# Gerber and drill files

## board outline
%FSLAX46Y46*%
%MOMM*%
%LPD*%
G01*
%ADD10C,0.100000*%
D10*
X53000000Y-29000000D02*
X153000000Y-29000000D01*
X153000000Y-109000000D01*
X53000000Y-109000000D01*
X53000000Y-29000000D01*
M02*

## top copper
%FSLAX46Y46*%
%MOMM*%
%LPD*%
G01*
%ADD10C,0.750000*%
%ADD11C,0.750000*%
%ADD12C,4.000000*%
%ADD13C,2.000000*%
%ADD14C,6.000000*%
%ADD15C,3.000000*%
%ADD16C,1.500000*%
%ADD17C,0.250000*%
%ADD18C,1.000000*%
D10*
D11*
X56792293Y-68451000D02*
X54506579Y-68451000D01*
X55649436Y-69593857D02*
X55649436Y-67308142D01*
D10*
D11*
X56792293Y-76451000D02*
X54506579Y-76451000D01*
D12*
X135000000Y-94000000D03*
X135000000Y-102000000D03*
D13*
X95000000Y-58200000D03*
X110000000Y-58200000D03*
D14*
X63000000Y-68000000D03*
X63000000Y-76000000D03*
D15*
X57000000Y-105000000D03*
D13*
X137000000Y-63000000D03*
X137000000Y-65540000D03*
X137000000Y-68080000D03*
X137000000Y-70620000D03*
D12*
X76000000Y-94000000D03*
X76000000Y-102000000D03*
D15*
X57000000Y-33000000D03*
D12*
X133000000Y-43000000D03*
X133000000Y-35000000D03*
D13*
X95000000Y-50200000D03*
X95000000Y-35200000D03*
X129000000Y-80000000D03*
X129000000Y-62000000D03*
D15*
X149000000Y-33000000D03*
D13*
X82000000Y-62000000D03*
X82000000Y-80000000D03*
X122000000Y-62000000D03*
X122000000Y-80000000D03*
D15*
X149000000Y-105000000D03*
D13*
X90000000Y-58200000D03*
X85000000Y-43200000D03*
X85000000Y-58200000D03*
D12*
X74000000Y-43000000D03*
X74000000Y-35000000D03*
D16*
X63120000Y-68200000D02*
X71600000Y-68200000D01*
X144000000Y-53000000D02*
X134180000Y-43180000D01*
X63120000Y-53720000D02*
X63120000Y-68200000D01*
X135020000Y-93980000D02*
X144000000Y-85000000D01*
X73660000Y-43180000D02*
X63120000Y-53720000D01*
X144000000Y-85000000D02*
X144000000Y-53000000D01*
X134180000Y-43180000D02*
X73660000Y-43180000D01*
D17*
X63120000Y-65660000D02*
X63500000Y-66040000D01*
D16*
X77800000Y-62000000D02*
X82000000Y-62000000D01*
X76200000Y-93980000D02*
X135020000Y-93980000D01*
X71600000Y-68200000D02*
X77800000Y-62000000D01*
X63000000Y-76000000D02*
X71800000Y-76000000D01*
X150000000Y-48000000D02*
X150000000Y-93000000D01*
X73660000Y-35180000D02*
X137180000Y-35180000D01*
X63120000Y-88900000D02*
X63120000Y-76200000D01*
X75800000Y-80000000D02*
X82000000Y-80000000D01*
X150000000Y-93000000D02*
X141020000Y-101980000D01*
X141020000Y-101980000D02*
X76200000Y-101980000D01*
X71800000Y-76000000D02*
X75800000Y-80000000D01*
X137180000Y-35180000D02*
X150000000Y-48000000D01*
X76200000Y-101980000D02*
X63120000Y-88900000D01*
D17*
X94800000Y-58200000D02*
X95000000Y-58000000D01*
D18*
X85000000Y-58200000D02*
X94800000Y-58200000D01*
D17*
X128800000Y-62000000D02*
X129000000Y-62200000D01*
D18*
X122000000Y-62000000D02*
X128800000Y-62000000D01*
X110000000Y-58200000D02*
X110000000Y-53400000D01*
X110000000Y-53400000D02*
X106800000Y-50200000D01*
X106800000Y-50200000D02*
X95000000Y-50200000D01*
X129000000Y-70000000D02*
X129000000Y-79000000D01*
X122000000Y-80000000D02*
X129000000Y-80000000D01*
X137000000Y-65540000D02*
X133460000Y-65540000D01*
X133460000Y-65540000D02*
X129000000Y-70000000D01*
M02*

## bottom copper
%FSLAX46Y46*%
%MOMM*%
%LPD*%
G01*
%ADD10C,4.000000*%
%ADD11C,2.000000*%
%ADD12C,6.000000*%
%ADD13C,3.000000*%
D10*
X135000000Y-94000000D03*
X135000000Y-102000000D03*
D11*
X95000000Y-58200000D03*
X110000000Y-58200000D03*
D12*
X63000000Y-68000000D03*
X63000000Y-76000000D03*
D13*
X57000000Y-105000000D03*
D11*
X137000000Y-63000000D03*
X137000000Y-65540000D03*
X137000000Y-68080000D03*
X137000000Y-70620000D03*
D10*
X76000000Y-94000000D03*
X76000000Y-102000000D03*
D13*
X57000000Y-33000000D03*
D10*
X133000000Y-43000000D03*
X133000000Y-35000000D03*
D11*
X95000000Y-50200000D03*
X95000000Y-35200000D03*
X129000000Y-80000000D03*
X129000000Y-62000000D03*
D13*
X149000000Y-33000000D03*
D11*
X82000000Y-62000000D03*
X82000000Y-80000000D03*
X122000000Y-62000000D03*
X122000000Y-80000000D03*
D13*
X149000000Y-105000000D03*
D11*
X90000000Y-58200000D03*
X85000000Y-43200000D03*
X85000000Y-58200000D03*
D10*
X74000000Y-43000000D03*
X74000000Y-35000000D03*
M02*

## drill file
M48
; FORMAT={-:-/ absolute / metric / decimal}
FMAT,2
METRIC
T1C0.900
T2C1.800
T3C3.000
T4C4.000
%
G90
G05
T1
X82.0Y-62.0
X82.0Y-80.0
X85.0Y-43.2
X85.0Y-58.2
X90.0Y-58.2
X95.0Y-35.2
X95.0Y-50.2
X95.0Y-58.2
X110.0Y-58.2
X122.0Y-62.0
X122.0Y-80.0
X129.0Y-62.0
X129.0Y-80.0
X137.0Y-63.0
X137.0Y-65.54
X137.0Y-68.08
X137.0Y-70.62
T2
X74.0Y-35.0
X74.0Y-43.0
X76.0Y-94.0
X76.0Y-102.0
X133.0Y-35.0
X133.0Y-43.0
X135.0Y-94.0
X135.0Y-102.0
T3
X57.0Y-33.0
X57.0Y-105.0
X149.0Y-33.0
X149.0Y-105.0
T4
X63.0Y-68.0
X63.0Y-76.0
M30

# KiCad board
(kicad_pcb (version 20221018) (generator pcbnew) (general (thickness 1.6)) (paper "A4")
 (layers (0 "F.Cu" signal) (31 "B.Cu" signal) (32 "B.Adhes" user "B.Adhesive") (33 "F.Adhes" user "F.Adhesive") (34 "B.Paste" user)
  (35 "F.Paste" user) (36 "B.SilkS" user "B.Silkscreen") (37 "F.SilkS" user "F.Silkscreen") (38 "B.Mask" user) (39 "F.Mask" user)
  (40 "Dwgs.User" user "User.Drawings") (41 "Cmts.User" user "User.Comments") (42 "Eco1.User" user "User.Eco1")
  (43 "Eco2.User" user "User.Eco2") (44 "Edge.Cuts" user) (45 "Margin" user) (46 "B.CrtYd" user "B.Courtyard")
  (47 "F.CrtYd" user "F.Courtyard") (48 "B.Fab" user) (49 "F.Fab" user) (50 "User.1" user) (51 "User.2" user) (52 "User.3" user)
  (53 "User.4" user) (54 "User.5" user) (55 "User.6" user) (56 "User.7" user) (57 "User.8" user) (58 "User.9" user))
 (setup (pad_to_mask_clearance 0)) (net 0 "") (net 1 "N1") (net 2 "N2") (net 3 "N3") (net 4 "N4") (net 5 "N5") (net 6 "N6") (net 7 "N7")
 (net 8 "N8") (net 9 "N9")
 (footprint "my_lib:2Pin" (layer "F.Cu") (at 135 94)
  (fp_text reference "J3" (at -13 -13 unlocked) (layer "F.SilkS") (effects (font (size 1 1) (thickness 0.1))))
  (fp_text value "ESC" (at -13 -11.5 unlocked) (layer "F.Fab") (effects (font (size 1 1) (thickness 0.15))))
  (pad "1" thru_hole circle (at 0 0) (size 4 4) (drill 1.8) (layers "*.Cu" "*.Mask") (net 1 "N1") (clearance 0.5))
  (pad "2" thru_hole circle (at 0 8) (size 4 4) (drill 1.8) (layers "*.Cu" "*.Mask") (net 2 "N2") (clearance 0.5)))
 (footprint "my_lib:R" (layer "F.Cu") (at 95 58.2)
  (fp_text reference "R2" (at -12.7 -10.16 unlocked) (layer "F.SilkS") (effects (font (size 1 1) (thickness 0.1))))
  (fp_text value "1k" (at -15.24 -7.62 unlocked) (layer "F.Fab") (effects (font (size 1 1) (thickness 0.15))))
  (pad "1" thru_hole circle (at 0 0) (size 2 2) (drill 0.9) (layers "*.Cu" "*.Mask") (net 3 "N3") (clearance 0.5))
  (pad "2" thru_hole circle (at 15 0) (size 2 2) (drill 0.9) (layers "*.Cu" "*.Mask") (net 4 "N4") (clearance 0.5)))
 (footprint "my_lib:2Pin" (layer "F.Cu") (at 63 68)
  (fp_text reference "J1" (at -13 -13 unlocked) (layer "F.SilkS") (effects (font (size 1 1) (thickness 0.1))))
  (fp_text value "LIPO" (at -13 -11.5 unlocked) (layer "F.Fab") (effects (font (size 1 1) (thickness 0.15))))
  (pad "1" thru_hole circle (at 0 0) (size 6 6) (drill 4) (layers "*.Cu" "*.Mask") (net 1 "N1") (clearance 0.5))
  (pad "2" thru_hole circle (at 0 8) (size 6 6) (drill 4) (layers "*.Cu" "*.Mask") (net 2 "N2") (clearance 0.5)))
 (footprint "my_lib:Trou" (layer "F.Cu") (at 57 105)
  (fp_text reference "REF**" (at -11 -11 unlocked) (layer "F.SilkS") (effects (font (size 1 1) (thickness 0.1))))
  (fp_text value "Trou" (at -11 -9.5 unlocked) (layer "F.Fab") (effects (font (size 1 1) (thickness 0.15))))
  (pad "1" thru_hole circle (at 0 0) (size 3 3) (drill 3) (layers "*.Cu" "*.Mask")))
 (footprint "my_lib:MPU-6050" (layer "F.Cu") (at 137 63)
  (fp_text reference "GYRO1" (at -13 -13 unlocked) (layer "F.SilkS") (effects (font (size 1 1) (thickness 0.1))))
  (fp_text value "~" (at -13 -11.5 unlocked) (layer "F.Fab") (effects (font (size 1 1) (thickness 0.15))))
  (pad "1" thru_hole circle (at 0 0) (size 2 2) (drill 0.9) (layers "*.Cu" "*.Mask") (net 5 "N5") (clearance 0.5))
  (pad "2" thru_hole circle (at 0 2.54) (size 2 2) (drill 0.9) (layers "*.Cu" "*.Mask") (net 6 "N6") (clearance 0.5))
  (pad "3" thru_hole circle (at 0 5.08) (size 2 2) (drill 0.9) (layers "*.Cu" "*.Mask") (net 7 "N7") (clearance 0.5))
  (pad "4" thru_hole circle (at 0 7.62) (size 2 2) (drill 0.9) (layers "*.Cu" "*.Mask") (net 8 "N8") (clearance 0.5)))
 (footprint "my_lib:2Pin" (layer "F.Cu") (at 76 94)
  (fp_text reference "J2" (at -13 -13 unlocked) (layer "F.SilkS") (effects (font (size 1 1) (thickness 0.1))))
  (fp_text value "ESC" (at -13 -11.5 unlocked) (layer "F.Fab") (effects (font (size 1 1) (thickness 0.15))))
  (pad "1" thru_hole circle (at 0 0) (size 4 4) (drill 1.8) (layers "*.Cu" "*.Mask") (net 1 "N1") (clearance 0.5))
  (pad "2" thru_hole circle (at 0 8) (size 4 4) (drill 1.8) (layers "*.Cu" "*.Mask") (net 2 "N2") (clearance 0.5)))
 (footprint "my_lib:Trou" (layer "F.Cu") (at 57 33)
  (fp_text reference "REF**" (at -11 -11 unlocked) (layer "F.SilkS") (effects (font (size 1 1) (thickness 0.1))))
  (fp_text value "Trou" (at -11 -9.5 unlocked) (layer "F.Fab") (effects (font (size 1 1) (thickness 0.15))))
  (pad "1" thru_hole circle (at 0 0) (size 3 3) (drill 3) (layers "*.Cu" "*.Mask")))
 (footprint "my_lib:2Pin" (layer "F.Cu") (at 133 43 180)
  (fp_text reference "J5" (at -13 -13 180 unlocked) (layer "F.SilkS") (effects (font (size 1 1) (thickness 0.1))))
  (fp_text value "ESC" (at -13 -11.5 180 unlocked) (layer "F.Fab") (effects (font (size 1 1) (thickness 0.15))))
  (pad "1" thru_hole circle (at 0 0 180) (size 4 4) (drill 1.8) (layers "*.Cu" "*.Mask") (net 1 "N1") (clearance 0.5))
  (pad "2" thru_hole circle (at 0 8 180) (size 4 4) (drill 1.8) (layers "*.Cu" "*.Mask") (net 2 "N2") (clearance 0.5)))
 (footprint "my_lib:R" (layer "F.Cu") (at 95 50.2 90)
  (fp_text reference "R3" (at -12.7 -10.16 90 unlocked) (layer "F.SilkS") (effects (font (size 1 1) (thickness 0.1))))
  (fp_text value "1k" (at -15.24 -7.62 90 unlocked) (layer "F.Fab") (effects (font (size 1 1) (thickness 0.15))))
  (pad "1" thru_hole circle (at 0 0 90) (size 2 2) (drill 0.9) (layers "*.Cu" "*.Mask") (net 4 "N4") (clearance 0.5))
  (pad "2" thru_hole circle (at 15 0 90) (size 2 2) (drill 0.9) (layers "*.Cu" "*.Mask") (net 2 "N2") (clearance 0.5)))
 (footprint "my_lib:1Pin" (layer "F.Cu") (at 129 80)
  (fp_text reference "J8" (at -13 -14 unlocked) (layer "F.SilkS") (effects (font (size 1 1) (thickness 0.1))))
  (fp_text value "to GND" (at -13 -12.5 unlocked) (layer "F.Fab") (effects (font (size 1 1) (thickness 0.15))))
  (pad "1" thru_hole circle (at 0 0) (size 2 2) (drill 0.9) (layers "*.Cu" "*.Mask") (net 6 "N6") (clearance 0.5)))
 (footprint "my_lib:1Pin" (layer "F.Cu") (at 129 62)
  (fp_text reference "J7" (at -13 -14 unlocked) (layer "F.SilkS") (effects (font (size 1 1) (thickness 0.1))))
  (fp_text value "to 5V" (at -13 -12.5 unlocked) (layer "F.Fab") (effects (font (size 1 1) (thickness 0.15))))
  (pad "1" thru_hole circle (at 0 0) (size 2 2) (drill 0.9) (layers "*.Cu" "*.Mask") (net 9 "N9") (clearance 0.5)))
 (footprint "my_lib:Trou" (layer "F.Cu") (at 149 33)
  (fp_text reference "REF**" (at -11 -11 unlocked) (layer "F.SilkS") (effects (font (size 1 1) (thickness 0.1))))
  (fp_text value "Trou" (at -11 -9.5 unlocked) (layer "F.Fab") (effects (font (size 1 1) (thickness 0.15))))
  (pad "1" thru_hole circle (at 0 0) (size 3 3) (drill 3) (layers "*.Cu" "*.Mask")))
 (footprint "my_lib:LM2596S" (layer "F.Cu") (at 82 62)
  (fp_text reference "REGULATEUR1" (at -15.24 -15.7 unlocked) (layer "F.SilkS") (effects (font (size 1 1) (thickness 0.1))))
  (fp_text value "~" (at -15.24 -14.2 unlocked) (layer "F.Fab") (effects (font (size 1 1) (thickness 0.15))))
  (pad "1" thru_hole circle (at 0 0) (size 2 2) (drill 0.9) (layers "*.Cu" "*.Mask") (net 1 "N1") (clearance 0.5))
  (pad "2" thru_hole circle (at 0 18) (size 2 2) (drill 0.9) (layers "*.Cu" "*.Mask") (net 2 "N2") (clearance 0.5))
  (pad "3" thru_hole circle (at 40 0) (size 2 2) (drill 0.9) (layers "*.Cu" "*.Mask") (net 9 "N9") (clearance 0.5))
  (pad "4" thru_hole circle (at 40 18) (size 2 2) (drill 0.9) (layers "*.Cu" "*.Mask") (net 6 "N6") (clearance 0.5)))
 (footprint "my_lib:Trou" (layer "F.Cu") (at 149 105)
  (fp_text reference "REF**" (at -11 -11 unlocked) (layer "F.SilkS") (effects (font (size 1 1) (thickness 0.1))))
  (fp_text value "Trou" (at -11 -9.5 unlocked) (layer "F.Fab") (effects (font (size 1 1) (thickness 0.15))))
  (pad "1" thru_hole circle (at 0 0) (size 3 3) (drill 3) (layers "*.Cu" "*.Mask")))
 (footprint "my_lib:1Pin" (layer "F.Cu") (at 90 58.2)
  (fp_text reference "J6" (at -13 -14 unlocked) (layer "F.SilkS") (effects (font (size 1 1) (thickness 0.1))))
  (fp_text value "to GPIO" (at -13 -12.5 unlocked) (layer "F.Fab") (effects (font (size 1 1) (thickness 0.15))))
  (pad "1" thru_hole circle (at 0 0) (size 2 2) (drill 0.9) (layers "*.Cu" "*.Mask") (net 3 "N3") (clearance 0.5)))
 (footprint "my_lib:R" (layer "B.Cu") (at 85 43.2 -90)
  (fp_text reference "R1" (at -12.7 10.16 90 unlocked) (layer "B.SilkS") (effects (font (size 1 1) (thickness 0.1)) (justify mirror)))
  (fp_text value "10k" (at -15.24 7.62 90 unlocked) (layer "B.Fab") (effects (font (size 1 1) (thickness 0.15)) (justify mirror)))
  (pad "1" thru_hole circle (at 0 0 270) (size 2 2) (drill 0.9) (layers "*.Cu" "*.Mask") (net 1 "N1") (clearance 0.5))
  (pad "2" thru_hole circle (at 15 0 270) (size 2 2) (drill 0.9) (layers "*.Cu" "*.Mask") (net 3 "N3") (clearance 0.5)))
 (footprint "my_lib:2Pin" (layer "B.Cu") (at 74 43)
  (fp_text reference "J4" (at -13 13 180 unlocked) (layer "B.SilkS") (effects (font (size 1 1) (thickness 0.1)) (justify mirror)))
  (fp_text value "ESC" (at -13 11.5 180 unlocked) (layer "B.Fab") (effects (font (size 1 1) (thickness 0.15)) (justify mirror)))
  (pad "1" thru_hole circle (at 0 0) (size 4 4) (drill 1.8) (layers "*.Cu" "*.Mask") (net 1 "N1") (clearance 0.5))
  (pad "2" thru_hole circle (at 0 -8) (size 4 4) (drill 1.8) (layers "*.Cu" "*.Mask") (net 2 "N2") (clearance 0.5)))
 (gr_rect (start 53 29) (end 153 109) (stroke (width 0.1) (type default)) (fill none) (layer "Edge.Cuts"))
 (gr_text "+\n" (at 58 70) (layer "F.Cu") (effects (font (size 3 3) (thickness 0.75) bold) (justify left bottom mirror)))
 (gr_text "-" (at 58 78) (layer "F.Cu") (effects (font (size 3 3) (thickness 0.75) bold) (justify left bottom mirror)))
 (segment (start 63.12 68.2) (end 71.6 68.2) (width 1.5) (layer "F.Cu") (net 1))
 (segment (start 144 53) (end 134.18 43.18) (width 1.5) (layer "F.Cu") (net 1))
 (segment (start 63.12 53.72) (end 63.12 68.2) (width 1.5) (layer "F.Cu") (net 1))
 (segment (start 135.02 93.98) (end 144 85) (width 1.5) (layer "F.Cu") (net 1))
 (segment (start 73.66 43.18) (end 63.12 53.72) (width 1.5) (layer "F.Cu") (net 1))
 (segment (start 144 85) (end 144 53) (width 1.5) (layer "F.Cu") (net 1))
 (segment (start 134.18 43.18) (end 73.66 43.18) (width 1.5) (layer "F.Cu") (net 1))
 (segment (start 63.12 65.66) (end 63.5 66.04) (width 0.25) (layer "F.Cu") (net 1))
 (segment (start 77.8 62) (end 82 62) (width 1.5) (layer "F.Cu") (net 1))
 (segment (start 76.2 93.98) (end 135.02 93.98) (width 1.5) (layer "F.Cu") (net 1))
 (segment (start 71.6 68.2) (end 77.8 62) (width 1.5) (layer "F.Cu") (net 1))
 (segment (start 63 76) (end 71.8 76) (width 1.5) (layer "F.Cu") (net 2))
 (segment (start 150 48) (end 150 93) (width 1.5) (layer "F.Cu") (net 2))
 (segment (start 73.66 35.18) (end 137.18 35.18) (width 1.5) (layer "F.Cu") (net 2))
 (segment (start 63.12 88.9) (end 63.12 76.2) (width 1.5) (layer "F.Cu") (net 2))
 (segment (start 75.8 80) (end 82 80) (width 1.5) (layer "F.Cu") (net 2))
 (segment (start 150 93) (end 141.02 101.98) (width 1.5) (layer "F.Cu") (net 2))
 (segment (start 141.02 101.98) (end 76.2 101.98) (width 1.5) (layer "F.Cu") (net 2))
 (segment (start 71.8 76) (end 75.8 80) (width 1.5) (layer "F.Cu") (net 2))
 (segment (start 137.18 35.18) (end 150 48) (width 1.5) (layer "F.Cu") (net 2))
 (segment (start 76.2 101.98) (end 63.12 88.9) (width 1.5) (layer "F.Cu") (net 2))
 (segment (start 94.8 58.2) (end 95 58) (width 0.25) (layer "F.Cu") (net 3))
 (segment (start 85 58.2) (end 94.8 58.2) (width 1) (layer "F.Cu") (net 3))
 (segment (start 128.8 62) (end 129 62.2) (width 0.25) (layer "F.Cu") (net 9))
 (segment (start 122 62) (end 128.8 62) (width 1) (layer "F.Cu") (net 9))
 (segment (start 110 58.2) (end 110 53.4) (width 1) (layer "F.Cu") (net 4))
 (segment (start 110 53.4) (end 106.8 50.2) (width 1) (layer "F.Cu") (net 4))
 (segment (start 106.8 50.2) (end 95 50.2) (width 1) (layer "F.Cu") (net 4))
 (segment (start 129 70) (end 129 79) (width 1) (layer "F.Cu") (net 6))
 (segment (start 122 80) (end 129 80) (width 1) (layer "F.Cu") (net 6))
 (segment (start 137 65.54) (end 133.46 65.54) (width 1) (layer "F.Cu") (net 6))
 (segment (start 133.46 65.54) (end 129 70) (width 1) (layer "F.Cu") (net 6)))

